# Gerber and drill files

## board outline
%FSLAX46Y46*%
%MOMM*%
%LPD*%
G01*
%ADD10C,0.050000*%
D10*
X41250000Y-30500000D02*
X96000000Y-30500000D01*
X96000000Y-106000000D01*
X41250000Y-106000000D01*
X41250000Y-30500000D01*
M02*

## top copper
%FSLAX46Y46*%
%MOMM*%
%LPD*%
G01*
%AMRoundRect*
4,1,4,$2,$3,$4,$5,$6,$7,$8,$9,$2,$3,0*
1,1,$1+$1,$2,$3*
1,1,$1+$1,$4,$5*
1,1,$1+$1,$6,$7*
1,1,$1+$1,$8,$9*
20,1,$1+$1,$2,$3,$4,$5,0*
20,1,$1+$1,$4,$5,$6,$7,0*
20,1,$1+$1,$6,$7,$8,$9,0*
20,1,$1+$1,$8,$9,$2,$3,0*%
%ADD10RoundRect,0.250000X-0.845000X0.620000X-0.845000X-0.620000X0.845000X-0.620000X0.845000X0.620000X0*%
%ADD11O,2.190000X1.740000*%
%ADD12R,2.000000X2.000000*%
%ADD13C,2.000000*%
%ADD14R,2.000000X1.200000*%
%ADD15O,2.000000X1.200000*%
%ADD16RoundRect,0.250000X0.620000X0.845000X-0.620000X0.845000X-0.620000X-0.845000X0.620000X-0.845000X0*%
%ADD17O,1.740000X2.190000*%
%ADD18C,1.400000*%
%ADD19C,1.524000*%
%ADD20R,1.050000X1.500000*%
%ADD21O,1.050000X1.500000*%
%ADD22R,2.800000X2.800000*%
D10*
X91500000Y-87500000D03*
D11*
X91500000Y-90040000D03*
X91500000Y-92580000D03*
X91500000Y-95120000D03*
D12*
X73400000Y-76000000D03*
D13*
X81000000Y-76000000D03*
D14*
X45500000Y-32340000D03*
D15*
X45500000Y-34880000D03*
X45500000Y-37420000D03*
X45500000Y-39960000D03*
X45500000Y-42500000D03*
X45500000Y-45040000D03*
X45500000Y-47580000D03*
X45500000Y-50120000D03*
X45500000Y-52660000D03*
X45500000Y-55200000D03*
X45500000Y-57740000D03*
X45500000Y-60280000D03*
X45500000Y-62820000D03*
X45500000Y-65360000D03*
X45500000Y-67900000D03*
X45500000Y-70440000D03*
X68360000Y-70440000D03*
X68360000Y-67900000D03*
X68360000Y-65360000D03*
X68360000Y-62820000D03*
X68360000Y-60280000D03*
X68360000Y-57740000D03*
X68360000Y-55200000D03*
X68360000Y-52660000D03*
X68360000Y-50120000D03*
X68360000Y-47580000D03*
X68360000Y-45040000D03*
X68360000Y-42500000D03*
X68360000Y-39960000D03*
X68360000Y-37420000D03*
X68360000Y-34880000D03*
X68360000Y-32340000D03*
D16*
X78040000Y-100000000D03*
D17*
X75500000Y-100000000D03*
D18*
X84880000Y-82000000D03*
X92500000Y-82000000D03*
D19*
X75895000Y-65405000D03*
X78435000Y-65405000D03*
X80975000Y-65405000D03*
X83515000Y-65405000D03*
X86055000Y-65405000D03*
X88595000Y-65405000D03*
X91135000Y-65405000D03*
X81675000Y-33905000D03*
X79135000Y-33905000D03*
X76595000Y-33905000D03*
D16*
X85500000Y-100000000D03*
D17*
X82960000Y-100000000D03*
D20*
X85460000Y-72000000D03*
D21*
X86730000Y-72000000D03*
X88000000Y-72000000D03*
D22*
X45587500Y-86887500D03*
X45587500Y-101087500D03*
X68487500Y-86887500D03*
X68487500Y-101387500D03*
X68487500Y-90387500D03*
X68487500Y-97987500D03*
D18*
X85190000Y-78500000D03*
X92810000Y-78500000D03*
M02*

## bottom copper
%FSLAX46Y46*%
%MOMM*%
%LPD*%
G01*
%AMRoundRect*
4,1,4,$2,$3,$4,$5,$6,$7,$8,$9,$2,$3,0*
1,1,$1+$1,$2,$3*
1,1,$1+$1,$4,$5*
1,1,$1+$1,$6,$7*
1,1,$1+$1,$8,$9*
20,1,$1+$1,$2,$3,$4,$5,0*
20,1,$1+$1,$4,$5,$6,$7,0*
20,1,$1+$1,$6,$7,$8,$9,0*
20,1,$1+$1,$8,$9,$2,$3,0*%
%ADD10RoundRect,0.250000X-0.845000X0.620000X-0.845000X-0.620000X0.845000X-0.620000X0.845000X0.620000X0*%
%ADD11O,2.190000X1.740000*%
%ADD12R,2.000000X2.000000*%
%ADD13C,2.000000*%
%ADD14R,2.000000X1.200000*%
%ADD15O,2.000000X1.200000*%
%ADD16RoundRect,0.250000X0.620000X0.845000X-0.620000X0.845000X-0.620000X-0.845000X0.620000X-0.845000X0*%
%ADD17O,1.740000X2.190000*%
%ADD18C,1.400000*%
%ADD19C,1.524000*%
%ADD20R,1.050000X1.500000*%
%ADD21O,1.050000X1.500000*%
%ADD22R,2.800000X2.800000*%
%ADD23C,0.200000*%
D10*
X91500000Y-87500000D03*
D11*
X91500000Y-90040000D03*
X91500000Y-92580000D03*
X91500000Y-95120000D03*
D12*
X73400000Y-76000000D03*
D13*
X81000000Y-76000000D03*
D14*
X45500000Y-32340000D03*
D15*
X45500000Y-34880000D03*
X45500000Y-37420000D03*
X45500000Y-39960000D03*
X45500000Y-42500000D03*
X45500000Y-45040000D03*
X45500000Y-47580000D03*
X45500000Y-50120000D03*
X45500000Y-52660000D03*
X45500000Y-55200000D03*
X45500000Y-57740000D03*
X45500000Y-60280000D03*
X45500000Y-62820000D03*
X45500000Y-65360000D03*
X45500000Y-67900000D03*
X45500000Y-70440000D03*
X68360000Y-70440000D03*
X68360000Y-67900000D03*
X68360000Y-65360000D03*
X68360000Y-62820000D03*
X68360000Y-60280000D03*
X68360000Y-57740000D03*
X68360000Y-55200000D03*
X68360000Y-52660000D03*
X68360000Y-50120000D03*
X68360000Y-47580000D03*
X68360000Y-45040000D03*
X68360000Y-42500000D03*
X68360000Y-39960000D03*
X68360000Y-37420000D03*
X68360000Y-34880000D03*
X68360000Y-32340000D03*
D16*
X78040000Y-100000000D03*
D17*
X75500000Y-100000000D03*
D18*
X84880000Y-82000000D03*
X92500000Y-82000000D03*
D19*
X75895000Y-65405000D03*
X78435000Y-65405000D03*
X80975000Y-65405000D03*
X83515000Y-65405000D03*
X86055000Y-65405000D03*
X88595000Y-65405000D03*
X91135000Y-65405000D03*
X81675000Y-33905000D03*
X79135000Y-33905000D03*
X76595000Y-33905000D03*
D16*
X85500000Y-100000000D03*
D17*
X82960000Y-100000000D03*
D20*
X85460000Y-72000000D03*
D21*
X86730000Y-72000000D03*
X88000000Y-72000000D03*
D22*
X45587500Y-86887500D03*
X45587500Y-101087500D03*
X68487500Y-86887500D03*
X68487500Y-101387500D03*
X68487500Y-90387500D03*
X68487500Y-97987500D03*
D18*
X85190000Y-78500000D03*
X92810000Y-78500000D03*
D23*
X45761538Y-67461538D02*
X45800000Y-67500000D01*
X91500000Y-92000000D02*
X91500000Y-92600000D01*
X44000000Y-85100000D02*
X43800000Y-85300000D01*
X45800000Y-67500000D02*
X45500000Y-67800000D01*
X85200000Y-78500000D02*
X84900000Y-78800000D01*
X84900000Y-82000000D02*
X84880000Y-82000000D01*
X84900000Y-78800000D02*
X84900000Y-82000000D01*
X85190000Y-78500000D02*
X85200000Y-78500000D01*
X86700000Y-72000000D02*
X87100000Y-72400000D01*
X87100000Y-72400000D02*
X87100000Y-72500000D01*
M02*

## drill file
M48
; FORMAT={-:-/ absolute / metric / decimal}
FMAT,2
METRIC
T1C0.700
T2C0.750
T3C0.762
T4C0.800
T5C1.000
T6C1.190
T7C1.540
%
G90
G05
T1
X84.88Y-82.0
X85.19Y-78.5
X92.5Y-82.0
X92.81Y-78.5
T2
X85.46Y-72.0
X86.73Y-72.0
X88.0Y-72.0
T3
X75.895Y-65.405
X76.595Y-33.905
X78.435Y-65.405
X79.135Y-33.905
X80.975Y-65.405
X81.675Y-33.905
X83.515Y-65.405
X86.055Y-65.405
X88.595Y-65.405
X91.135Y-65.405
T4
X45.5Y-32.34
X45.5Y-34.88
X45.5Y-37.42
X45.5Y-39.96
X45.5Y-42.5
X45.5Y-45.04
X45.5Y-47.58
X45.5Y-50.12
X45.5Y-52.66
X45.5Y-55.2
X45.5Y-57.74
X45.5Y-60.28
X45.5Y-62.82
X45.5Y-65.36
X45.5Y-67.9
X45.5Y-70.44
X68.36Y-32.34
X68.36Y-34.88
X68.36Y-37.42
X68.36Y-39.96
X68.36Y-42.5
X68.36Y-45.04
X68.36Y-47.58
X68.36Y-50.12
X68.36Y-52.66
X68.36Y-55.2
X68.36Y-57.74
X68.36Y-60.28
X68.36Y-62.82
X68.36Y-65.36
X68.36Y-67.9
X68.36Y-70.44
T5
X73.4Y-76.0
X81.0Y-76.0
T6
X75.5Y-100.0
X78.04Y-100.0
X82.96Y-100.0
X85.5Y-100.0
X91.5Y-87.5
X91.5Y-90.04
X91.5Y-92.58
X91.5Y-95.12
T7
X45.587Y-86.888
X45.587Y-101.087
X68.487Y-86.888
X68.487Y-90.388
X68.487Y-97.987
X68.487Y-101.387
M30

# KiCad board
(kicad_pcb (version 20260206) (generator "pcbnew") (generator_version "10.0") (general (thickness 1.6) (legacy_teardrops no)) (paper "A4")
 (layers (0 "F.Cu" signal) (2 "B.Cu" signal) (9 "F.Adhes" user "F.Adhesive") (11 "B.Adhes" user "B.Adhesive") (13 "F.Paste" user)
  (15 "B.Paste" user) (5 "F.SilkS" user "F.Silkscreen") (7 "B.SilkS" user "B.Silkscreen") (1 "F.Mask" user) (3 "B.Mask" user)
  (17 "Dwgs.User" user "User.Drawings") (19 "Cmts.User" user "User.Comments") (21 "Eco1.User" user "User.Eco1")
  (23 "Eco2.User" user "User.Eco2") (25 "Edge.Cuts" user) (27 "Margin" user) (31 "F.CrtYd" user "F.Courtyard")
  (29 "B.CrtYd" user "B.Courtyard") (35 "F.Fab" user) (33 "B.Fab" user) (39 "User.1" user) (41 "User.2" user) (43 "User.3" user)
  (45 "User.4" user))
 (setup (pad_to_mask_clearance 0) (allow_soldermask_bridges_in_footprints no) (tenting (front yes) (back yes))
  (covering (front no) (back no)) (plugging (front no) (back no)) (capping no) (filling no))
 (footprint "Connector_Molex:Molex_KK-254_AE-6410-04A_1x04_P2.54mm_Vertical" (layer "F.Cu") (at 91.5 87.5 -90)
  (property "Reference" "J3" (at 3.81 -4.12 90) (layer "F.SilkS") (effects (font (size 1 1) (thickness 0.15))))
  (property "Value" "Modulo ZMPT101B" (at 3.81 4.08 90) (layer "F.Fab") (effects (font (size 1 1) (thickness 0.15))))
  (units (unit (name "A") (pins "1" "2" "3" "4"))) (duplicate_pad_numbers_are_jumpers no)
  (pad "1" thru_hole roundrect (at 0 0 270) (size 1.74 2.19) (drill 1.19) (layers "*.Cu" "*.Mask") (remove_unused_layers no)
   (roundrect_rratio 0.143678) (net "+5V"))
  (pad "2" thru_hole oval (at 2.54 0 270) (size 1.74 2.19) (drill 1.19) (layers "*.Cu" "*.Mask") (remove_unused_layers no)
   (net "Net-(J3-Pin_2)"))
  (pad "3" thru_hole oval (at 5.08 0 270) (size 1.74 2.19) (drill 1.19) (layers "*.Cu" "*.Mask") (remove_unused_layers no) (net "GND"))
  (pad "4" thru_hole oval (at 7.62 0 270) (size 1.74 2.19) (drill 1.19) (layers "*.Cu" "*.Mask") (remove_unused_layers no) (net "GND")))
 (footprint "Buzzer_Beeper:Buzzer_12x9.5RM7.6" (layer "F.Cu") (at 73.4 76)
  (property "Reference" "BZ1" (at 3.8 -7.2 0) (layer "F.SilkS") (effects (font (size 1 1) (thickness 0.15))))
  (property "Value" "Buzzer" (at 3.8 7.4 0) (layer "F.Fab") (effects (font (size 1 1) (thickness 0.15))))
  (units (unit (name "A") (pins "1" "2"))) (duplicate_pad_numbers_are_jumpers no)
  (pad "1" thru_hole rect (at 0 0) (size 2 2) (drill 1) (layers "*.Cu" "*.Mask") (remove_unused_layers no) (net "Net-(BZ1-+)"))
  (pad "2" thru_hole circle (at 7.6 0) (size 2 2) (drill 1) (layers "*.Cu" "*.Mask") (remove_unused_layers no) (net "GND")))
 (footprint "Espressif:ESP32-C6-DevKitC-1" (layer "F.Cu") (at 45.5 32.34)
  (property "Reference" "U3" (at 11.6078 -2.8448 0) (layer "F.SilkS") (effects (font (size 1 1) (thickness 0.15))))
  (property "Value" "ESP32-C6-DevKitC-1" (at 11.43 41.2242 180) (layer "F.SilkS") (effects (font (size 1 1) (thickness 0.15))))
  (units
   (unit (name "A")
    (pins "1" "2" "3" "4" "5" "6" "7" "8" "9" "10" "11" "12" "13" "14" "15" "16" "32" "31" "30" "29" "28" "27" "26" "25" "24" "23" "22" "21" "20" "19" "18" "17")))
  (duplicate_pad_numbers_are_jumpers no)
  (pad "1" thru_hole rect (at 0 0 270) (size 1.2 2) (drill 0.8) (layers "*.Cu" "*.Mask") (remove_unused_layers no)
   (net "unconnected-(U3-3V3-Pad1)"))
  (pad "2" thru_hole oval (at 0 2.54 270) (size 1.2 2) (drill 0.8) (layers "*.Cu" "*.Mask") (remove_unused_layers no)
   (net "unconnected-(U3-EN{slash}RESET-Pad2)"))
  (pad "3" thru_hole oval (at 0 5.08 270) (size 1.2 2) (drill 0.8) (layers "*.Cu" "*.Mask") (remove_unused_layers no)
   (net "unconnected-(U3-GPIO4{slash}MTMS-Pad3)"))
  (pad "4" thru_hole oval (at 0 7.62 270) (size 1.2 2) (drill 0.8) (layers "*.Cu" "*.Mask") (remove_unused_layers no)
   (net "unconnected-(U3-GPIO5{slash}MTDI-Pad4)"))
  (pad "5" thru_hole oval (at 0 10.16 270) (size 1.2 2) (drill 0.8) (layers "*.Cu" "*.Mask") (remove_unused_layers no)
   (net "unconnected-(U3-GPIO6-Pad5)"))
  (pad "6" thru_hole oval (at 0 12.7 270) (size 1.2 2) (drill 0.8) (layers "*.Cu" "*.Mask") (remove_unused_layers no)
   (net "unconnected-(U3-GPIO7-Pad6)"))
  (pad "7" thru_hole oval (at 0 15.24 270) (size 1.2 2) (drill 0.8) (layers "*.Cu" "*.Mask") (remove_unused_layers no)
   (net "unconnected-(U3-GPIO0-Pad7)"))
  (pad "8" thru_hole oval (at 0 17.78 270) (size 1.2 2) (drill 0.8) (layers "*.Cu" "*.Mask") (remove_unused_layers no)
   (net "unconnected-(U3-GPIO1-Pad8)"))
  (pad "9" thru_hole oval (at 0 20.32 270) (size 1.2 2) (drill 0.8) (layers "*.Cu" "*.Mask") (remove_unused_layers no)
   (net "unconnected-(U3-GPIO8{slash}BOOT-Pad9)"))
  (pad "10" thru_hole oval (at 0 22.86 270) (size 1.2 2) (drill 0.8) (layers "*.Cu" "*.Mask") (remove_unused_layers no)
   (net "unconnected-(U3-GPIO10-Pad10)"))
  (pad "11" thru_hole oval (at 0 25.4 270) (size 1.2 2) (drill 0.8) (layers "*.Cu" "*.Mask") (remove_unused_layers no)
   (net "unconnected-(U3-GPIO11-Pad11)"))
  (pad "12" thru_hole oval (at 0 27.94 270) (size 1.2 2) (drill 0.8) (layers "*.Cu" "*.Mask") (remove_unused_layers no)
   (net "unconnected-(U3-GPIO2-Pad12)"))
  (pad "13" thru_hole oval (at 0 30.48 270) (size 1.2 2) (drill 0.8) (layers "*.Cu" "*.Mask") (remove_unused_layers no)
   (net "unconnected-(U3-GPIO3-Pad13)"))
  (pad "14" thru_hole oval (at 0 33.02 270) (size 1.2 2) (drill 0.8) (layers "*.Cu" "*.Mask") (remove_unused_layers no) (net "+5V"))
  (pad "15" thru_hole oval (at 0 35.56 270) (size 1.2 2) (drill 0.8) (layers "*.Cu" "*.Mask") (remove_unused_layers no) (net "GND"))
  (pad "16" thru_hole oval (at 0 38.1 270) (size 1.2 2) (drill 0.8) (layers "*.Cu" "*.Mask") (remove_unused_layers no)
   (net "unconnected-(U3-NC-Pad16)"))
  (pad "17" thru_hole oval (at 22.86 38.1 270) (size 1.2 2) (drill 0.8) (layers "*.Cu" "*.Mask") (remove_unused_layers no)
   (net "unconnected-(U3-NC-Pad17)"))
  (pad "18" thru_hole oval (at 22.86 35.56 270) (size 1.2 2) (drill 0.8) (layers "*.Cu" "*.Mask") (remove_unused_layers no) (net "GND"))
  (pad "19" thru_hole oval (at 22.86 33.02 270) (size 1.2 2) (drill 0.8) (layers "*.Cu" "*.Mask") (remove_unused_layers no)
   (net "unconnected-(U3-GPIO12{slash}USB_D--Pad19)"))
  (pad "20" thru_hole oval (at 22.86 30.48 270) (size 1.2 2) (drill 0.8) (layers "*.Cu" "*.Mask") (remove_unused_layers no)
   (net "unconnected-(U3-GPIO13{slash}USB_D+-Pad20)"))
  (pad "21" thru_hole oval (at 22.86 27.94 270) (size 1.2 2) (drill 0.8) (layers "*.Cu" "*.Mask") (remove_unused_layers no) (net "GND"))
  (pad "22" thru_hole oval (at 22.86 25.4 270) (size 1.2 2) (drill 0.8) (layers "*.Cu" "*.Mask") (remove_unused_layers no)
   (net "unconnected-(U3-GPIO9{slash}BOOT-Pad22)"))
  (pad "23" thru_hole oval (at 22.86 22.86 270) (size 1.2 2) (drill 0.8) (layers "*.Cu" "*.Mask") (remove_unused_layers no)
   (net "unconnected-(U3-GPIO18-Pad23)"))
  (pad "24" thru_hole oval (at 22.86 20.32 270) (size 1.2 2) (drill 0.8) (layers "*.Cu" "*.Mask") (remove_unused_layers no)
   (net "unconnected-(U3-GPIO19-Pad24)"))
  (pad "25" thru_hole oval (at 22.86 17.78 270) (size 1.2 2) (drill 0.8) (layers "*.Cu" "*.Mask") (remove_unused_layers no)
   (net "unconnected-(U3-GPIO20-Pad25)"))
  (pad "26" thru_hole oval (at 22.86 15.24 270) (size 1.2 2) (drill 0.8) (layers "*.Cu" "*.Mask") (remove_unused_layers no) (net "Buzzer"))
  (pad "27" thru_hole oval (at 22.86 12.7 270) (size 1.2 2) (drill 0.8) (layers "*.Cu" "*.Mask") (remove_unused_layers no)
   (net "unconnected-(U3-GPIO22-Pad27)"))
  (pad "28" thru_hole oval (at 22.86 10.16 270) (size 1.2 2) (drill 0.8) (layers "*.Cu" "*.Mask") (remove_unused_layers no)
   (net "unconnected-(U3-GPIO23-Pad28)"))
  (pad "29" thru_hole oval (at 22.86 7.62 270) (size 1.2 2) (drill 0.8) (layers "*.Cu" "*.Mask") (remove_unused_layers no)
   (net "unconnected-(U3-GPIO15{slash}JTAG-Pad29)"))
  (pad "30" thru_hole oval (at 22.86 5.08 270) (size 1.2 2) (drill 0.8) (layers "*.Cu" "*.Mask") (remove_unused_layers no)
   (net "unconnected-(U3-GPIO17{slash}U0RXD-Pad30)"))
  (pad "31" thru_hole oval (at 22.86 2.54 270) (size 1.2 2) (drill 0.8) (layers "*.Cu" "*.Mask") (remove_unused_layers no)
   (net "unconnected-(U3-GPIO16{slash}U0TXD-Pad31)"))
  (pad "32" thru_hole oval (at 22.86 0 270) (size 1.2 2) (drill 0.8) (layers "*.Cu" "*.Mask") (remove_unused_layers no) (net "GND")))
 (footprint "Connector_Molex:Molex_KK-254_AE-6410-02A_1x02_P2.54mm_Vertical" (layer "F.Cu") (at 78.04 100 180)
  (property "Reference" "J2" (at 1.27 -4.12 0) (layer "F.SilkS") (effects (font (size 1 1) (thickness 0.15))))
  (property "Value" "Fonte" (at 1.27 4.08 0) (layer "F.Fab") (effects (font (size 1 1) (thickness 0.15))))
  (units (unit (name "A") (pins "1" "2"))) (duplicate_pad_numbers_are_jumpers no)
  (pad "1" thru_hole roundrect (at 0 0 180) (size 1.74 2.19) (drill 1.19) (layers "*.Cu" "*.Mask") (remove_unused_layers no)
   (roundrect_rratio 0.143678) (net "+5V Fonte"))
  (pad "2" thru_hole oval (at 2.54 0 180) (size 1.74 2.19) (drill 1.19) (layers "*.Cu" "*.Mask") (remove_unused_layers no) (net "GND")))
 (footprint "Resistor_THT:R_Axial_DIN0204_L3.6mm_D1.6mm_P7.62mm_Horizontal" (layer "F.Cu") (at 84.88 82)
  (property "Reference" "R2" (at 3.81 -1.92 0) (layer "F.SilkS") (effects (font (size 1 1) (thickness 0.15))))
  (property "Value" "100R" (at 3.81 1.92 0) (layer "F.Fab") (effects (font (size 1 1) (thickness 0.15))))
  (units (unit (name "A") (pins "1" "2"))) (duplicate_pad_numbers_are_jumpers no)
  (pad "1" thru_hole circle (at 0 0) (size 1.4 1.4) (drill 0.7) (layers "*.Cu" "*.Mask") (remove_unused_layers no) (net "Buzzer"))
  (pad "2" thru_hole circle (at 7.62 0) (size 1.4 1.4) (drill 0.7) (layers "*.Cu" "*.Mask") (remove_unused_layers no) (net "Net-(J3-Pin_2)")))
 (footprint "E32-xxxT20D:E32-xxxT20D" (layer "F.Cu") (at 73.095 66.905 90)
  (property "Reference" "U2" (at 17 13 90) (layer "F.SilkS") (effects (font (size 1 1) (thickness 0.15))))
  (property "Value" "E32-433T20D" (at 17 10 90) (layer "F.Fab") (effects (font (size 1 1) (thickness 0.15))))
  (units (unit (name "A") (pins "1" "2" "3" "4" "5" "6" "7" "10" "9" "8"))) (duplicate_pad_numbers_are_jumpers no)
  (pad "1" thru_hole circle (at 1.5 2.8 90) (size 1.524 1.524) (drill 0.762) (layers "*.Cu" "*.Mask") (remove_unused_layers no)
   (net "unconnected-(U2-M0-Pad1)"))
  (pad "2" thru_hole circle (at 1.5 5.34 90) (size 1.524 1.524) (drill 0.762) (layers "*.Cu" "*.Mask") (remove_unused_layers no)
   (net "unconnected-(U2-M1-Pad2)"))
  (pad "3" thru_hole circle (at 1.5 7.88 90) (size 1.524 1.524) (drill 0.762) (layers "*.Cu" "*.Mask") (remove_unused_layers no)
   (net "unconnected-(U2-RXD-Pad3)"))
  (pad "4" thru_hole circle (at 1.5 10.42 90) (size 1.524 1.524) (drill 0.762) (layers "*.Cu" "*.Mask") (remove_unused_layers no)
   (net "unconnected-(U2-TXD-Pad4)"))
  (pad "5" thru_hole circle (at 1.5 12.96 90) (size 1.524 1.524) (drill 0.762) (layers "*.Cu" "*.Mask") (remove_unused_layers no)
   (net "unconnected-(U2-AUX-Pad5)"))
  (pad "6" thru_hole circle (at 1.5 15.5 90) (size 1.524 1.524) (drill 0.762) (layers "*.Cu" "*.Mask") (remove_unused_layers no) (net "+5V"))
  (pad "7" thru_hole circle (at 1.5 18.04 90) (size 1.524 1.524) (drill 0.762) (layers "*.Cu" "*.Mask") (remove_unused_layers no)
   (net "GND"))
  (pad "8" thru_hole circle (at 33 8.58 90) (size 1.524 1.524) (drill 0.762) (layers "*.Cu" "*.Mask") (remove_unused_layers no)
   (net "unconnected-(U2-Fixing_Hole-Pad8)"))
  (pad "9" thru_hole circle (at 33 6.04 90) (size 1.524 1.524) (drill 0.762) (layers "*.Cu" "*.Mask") (remove_unused_layers no)
   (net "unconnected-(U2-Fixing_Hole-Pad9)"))
  (pad "10" thru_hole circle (at 33 3.5 90) (size 1.524 1.524) (drill 0.762) (layers "*.Cu" "*.Mask") (remove_unused_layers no)
   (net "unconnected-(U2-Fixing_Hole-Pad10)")))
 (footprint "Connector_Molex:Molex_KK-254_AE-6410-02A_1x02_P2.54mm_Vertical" (layer "F.Cu") (at 85.5 100 180)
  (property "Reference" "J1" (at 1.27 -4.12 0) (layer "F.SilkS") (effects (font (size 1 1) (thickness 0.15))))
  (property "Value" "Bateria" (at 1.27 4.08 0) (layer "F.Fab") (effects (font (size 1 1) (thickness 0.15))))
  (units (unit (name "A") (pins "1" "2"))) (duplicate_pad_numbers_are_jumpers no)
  (pad "1" thru_hole roundrect (at 0 0 180) (size 1.74 2.19) (drill 1.19) (layers "*.Cu" "*.Mask") (remove_unused_layers no)
   (roundrect_rratio 0.143678) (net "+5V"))
  (pad "2" thru_hole oval (at 2.54 0 180) (size 1.74 2.19) (drill 1.19) (layers "*.Cu" "*.Mask") (remove_unused_layers no) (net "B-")))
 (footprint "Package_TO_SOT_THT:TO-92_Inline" (layer "F.Cu") (at 85.46 72)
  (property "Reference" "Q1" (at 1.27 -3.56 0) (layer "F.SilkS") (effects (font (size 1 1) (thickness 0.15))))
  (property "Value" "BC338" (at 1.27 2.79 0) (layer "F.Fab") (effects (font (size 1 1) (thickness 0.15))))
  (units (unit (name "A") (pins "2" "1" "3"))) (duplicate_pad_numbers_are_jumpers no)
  (pad "1" thru_hole rect (at 0 0) (size 1.05 1.5) (drill 0.75) (layers "*.Cu" "*.Mask") (remove_unused_layers no) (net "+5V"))
  (pad "2" thru_hole oval (at 1.27 0) (size 1.05 1.5) (drill 0.75) (layers "*.Cu" "*.Mask") (remove_unused_layers no) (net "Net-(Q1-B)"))
  (pad "3" thru_hole oval (at 2.54 0) (size 1.05 1.5) (drill 0.75) (layers "*.Cu" "*.Mask") (remove_unused_layers no) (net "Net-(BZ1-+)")))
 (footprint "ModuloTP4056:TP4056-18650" (layer "F.Cu") (at 43.8875 85.1875)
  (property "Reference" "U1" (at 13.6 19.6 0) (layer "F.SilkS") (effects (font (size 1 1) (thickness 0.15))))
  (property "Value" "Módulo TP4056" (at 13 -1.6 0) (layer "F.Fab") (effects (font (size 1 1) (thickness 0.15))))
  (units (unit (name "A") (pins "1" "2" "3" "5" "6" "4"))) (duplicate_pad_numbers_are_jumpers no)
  (pad "1" thru_hole rect (at 1.7 1.7) (size 2.8 2.8) (drill 1.54) (layers "*.Cu" "*.Mask") (remove_unused_layers no) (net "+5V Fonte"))
  (pad "2" thru_hole rect (at 1.7 15.9) (size 2.8 2.8) (drill 1.54) (layers "*.Cu" "*.Mask") (remove_unused_layers no) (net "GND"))
  (pad "3" thru_hole rect (at 24.6 1.7) (size 2.8 2.8) (drill 1.54) (layers "*.Cu" "*.Mask") (remove_unused_layers no) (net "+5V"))
  (pad "4" thru_hole rect (at 24.6 16.2) (size 2.8 2.8) (drill 1.54) (layers "*.Cu" "*.Mask") (remove_unused_layers no) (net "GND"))
  (pad "5" thru_hole rect (at 24.6 5.2) (size 2.8 2.8) (drill 1.54) (layers "*.Cu" "*.Mask") (remove_unused_layers no) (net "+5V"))
  (pad "6" thru_hole rect (at 24.6 12.8) (size 2.8 2.8) (drill 1.54) (layers "*.Cu" "*.Mask") (remove_unused_layers no) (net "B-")))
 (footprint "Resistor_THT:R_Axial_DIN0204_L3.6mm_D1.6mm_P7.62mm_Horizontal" (layer "F.Cu") (at 85.19 78.5)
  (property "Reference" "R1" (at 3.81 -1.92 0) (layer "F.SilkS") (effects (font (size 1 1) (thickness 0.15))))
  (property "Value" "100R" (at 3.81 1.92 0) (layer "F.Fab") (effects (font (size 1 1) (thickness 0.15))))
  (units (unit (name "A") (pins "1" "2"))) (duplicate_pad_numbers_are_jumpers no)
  (pad "1" thru_hole circle (at 0 0) (size 1.4 1.4) (drill 0.7) (layers "*.Cu" "*.Mask") (remove_unused_layers no) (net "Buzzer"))
  (pad "2" thru_hole circle (at 7.62 0) (size 1.4 1.4) (drill 0.7) (layers "*.Cu" "*.Mask") (remove_unused_layers no) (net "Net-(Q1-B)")))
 (gr_rect (start 41.25 30.5) (end 96 106) (stroke (width 0.05) (type default)) (fill no) (layer "Edge.Cuts"))
 (segment (start 45.761538 67.461538) (end 45.8 67.5) (width 0.2) (layer "B.Cu") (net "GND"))
 (segment (start 91.5 92) (end 91.5 92.6) (width 0.2) (layer "B.Cu") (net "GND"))
 (segment (start 44 85.1) (end 43.8 85.3) (width 0.2) (layer "B.Cu") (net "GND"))
 (segment (start 45.8 67.5) (end 45.5 67.8) (width 0.2) (layer "B.Cu") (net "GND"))
 (segment (start 85.2 78.5) (end 84.9 78.8) (width 0.2) (layer "B.Cu") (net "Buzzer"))
 (segment (start 84.9 82) (end 84.88 82) (width 0.2) (layer "B.Cu") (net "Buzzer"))
 (segment (start 84.9 78.8) (end 84.9 82) (width 0.2) (layer "B.Cu") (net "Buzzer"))
 (segment (start 85.19 78.5) (end 85.2 78.5) (width 0.2) (layer "B.Cu") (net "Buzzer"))
 (segment (start 86.7 72) (end 87.1 72.4) (width 0.2) (layer "B.Cu") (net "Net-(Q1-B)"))
 (segment (start 87.1 72.4) (end 87.1 72.5) (width 0.2) (layer "B.Cu") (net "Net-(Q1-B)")))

